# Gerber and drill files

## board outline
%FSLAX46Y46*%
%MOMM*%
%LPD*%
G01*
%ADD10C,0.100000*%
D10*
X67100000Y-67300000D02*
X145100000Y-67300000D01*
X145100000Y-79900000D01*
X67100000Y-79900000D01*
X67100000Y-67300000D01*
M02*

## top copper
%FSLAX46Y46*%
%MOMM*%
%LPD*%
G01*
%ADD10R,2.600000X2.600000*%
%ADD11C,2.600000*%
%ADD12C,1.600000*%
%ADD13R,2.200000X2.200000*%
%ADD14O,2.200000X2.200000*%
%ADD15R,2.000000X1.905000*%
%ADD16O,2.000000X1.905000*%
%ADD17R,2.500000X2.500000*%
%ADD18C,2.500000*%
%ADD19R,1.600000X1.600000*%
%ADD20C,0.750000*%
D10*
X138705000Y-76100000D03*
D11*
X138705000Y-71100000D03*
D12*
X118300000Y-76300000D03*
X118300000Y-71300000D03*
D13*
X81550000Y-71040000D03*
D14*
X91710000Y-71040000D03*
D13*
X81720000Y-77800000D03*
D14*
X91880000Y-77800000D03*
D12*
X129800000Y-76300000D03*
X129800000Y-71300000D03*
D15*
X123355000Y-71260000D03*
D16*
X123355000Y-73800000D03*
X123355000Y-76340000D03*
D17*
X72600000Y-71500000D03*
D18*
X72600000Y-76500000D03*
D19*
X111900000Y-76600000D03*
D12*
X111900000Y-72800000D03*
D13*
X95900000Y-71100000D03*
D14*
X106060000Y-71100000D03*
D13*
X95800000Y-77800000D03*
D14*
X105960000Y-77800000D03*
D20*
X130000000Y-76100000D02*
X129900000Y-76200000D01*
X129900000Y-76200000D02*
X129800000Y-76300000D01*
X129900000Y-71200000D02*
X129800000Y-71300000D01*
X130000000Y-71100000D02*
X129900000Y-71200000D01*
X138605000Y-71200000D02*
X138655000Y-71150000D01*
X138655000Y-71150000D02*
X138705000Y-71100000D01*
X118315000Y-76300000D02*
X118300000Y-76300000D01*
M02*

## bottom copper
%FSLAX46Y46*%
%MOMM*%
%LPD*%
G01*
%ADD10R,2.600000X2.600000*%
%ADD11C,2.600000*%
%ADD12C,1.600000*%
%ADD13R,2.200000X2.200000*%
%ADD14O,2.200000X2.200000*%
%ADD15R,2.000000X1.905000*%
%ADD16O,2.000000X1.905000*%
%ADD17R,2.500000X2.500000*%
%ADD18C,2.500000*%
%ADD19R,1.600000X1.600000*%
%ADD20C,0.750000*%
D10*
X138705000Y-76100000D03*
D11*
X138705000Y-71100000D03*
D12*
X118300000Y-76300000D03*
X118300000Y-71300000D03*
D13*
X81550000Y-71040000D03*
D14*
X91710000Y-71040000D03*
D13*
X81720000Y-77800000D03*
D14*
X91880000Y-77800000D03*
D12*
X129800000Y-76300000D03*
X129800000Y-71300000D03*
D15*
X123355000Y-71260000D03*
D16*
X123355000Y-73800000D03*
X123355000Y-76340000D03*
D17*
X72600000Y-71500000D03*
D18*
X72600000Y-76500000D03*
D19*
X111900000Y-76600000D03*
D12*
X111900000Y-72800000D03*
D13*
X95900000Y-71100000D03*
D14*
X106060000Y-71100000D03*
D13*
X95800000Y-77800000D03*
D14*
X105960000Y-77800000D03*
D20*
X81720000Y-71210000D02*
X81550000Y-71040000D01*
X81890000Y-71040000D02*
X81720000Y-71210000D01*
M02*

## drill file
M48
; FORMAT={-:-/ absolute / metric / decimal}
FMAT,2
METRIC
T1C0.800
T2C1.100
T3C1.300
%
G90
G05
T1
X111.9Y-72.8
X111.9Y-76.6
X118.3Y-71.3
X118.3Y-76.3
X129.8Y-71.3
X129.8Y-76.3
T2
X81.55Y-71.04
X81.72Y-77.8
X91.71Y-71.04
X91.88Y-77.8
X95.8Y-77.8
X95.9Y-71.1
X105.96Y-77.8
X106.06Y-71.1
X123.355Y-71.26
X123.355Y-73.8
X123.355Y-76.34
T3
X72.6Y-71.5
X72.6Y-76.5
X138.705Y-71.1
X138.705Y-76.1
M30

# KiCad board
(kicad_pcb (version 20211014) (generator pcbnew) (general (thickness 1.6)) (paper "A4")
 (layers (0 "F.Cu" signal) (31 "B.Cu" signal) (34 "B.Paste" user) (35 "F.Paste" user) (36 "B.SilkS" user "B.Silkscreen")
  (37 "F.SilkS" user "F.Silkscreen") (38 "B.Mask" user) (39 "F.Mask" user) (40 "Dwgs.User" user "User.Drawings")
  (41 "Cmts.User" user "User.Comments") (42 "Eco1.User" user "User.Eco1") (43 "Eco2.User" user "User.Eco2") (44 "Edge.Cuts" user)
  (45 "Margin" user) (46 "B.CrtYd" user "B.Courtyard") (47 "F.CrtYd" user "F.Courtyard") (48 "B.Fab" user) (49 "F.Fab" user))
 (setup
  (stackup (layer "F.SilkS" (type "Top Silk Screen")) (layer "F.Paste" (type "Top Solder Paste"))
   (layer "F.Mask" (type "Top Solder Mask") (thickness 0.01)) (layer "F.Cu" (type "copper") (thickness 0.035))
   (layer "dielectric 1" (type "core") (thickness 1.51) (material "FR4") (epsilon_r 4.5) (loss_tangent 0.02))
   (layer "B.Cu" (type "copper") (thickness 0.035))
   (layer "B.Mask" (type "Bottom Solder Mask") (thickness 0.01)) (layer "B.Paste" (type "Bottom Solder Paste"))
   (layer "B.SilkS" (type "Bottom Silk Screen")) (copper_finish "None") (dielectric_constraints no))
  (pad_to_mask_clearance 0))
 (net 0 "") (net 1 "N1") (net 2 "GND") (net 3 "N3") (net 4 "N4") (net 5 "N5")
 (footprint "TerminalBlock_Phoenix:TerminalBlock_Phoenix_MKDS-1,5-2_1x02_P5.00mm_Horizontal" (layer "F.Cu") (at 138.705 76.1 90)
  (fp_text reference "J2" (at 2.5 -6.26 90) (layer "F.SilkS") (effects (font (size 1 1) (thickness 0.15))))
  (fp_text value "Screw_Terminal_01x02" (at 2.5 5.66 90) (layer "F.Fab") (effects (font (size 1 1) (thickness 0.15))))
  (pad "1" thru_hole rect (at 0 0 90) (size 2.6 2.6) (drill 1.3) (layers *.Cu *.Mask) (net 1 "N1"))
  (pad "2" thru_hole circle (at 5 0 90) (size 2.6 2.6) (drill 1.3) (layers *.Cu *.Mask) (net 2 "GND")))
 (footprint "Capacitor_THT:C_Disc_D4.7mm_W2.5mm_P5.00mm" (layer "F.Cu") (at 118.3 76.3 90)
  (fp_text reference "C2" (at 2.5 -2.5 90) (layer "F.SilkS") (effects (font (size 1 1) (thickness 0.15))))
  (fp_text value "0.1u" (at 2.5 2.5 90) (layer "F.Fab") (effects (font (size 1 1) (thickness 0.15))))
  (pad "1" thru_hole circle (at 0 0 90) (size 1.6 1.6) (drill 0.8) (layers *.Cu *.Mask) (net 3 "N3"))
  (pad "2" thru_hole circle (at 5 0 90) (size 1.6 1.6) (drill 0.8) (layers *.Cu *.Mask) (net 2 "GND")))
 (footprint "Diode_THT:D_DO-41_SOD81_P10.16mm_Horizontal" (layer "F.Cu") (at 81.55 71.04)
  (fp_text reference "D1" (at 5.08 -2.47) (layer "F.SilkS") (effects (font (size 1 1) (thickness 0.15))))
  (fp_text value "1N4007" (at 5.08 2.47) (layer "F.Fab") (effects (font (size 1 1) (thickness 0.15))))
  (pad "1" thru_hole rect (at 0 0) (size 2.2 2.2) (drill 1.1) (layers *.Cu *.Mask) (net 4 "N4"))
  (pad "2" thru_hole oval (at 10.16 0) (size 2.2 2.2) (drill 1.1) (layers *.Cu *.Mask) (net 2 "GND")))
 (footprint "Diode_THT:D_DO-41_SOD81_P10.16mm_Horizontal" (layer "F.Cu") (at 81.72 77.8)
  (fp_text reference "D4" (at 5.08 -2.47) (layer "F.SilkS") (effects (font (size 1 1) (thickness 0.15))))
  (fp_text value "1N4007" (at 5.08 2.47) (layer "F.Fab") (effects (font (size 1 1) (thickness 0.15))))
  (pad "1" thru_hole rect (at 0 0) (size 2.2 2.2) (drill 1.1) (layers *.Cu *.Mask) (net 3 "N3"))
  (pad "2" thru_hole oval (at 10.16 0) (size 2.2 2.2) (drill 1.1) (layers *.Cu *.Mask) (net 4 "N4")))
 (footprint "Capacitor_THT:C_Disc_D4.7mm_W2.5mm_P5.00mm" (layer "F.Cu") (at 129.8 76.3 90)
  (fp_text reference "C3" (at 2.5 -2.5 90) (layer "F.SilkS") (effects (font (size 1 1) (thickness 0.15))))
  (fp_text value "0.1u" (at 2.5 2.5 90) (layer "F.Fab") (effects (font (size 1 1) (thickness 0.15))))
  (pad "1" thru_hole circle (at 0 0 90) (size 1.6 1.6) (drill 0.8) (layers *.Cu *.Mask) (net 1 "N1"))
  (pad "2" thru_hole circle (at 5 0 90) (size 1.6 1.6) (drill 0.8) (layers *.Cu *.Mask) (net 2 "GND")))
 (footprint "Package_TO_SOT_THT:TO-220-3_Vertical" (layer "F.Cu") (at 123.355 71.26 -90)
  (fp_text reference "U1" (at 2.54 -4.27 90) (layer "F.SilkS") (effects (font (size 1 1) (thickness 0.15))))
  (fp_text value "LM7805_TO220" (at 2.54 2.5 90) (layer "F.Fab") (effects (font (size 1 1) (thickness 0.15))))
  (pad "1" thru_hole rect (at 0 0 270) (size 1.905 2) (drill 1.1) (layers *.Cu *.Mask) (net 3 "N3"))
  (pad "2" thru_hole oval (at 2.54 0 270) (size 1.905 2) (drill 1.1) (layers *.Cu *.Mask) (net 2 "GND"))
  (pad "3" thru_hole oval (at 5.08 0 270) (size 1.905 2) (drill 1.1) (layers *.Cu *.Mask) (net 1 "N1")))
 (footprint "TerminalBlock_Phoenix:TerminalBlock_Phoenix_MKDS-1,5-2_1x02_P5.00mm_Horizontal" (layer "F.Cu") (at 72.6 71.5 -90)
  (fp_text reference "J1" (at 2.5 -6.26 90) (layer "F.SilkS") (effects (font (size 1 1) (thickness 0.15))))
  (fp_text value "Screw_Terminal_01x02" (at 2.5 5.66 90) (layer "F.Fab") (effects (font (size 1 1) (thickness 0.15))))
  (pad "1" thru_hole rect (at 0 0 270) (size 2.5 2.5) (drill 1.3) (layers *.Cu *.Mask) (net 4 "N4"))
  (pad "2" thru_hole circle (at 5 0 270) (size 2.5 2.5) (drill 1.3) (layers *.Cu *.Mask) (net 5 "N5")))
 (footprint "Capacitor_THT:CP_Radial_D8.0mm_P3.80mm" (layer "F.Cu") (at 111.9 76.6 90)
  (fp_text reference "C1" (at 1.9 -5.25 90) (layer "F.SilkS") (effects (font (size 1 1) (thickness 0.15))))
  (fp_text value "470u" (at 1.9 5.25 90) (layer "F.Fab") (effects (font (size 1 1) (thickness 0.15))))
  (pad "1" thru_hole rect (at 0 0 90) (size 1.6 1.6) (drill 0.8) (layers *.Cu *.Mask) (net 3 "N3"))
  (pad "2" thru_hole circle (at 3.8 0 90) (size 1.6 1.6) (drill 0.8) (layers *.Cu *.Mask) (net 2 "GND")))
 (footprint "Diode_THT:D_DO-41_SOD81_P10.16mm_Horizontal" (layer "F.Cu") (at 95.9 71.1)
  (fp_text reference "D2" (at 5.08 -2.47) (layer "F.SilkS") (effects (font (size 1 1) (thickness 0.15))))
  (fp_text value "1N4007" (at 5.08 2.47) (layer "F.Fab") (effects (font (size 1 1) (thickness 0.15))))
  (pad "1" thru_hole rect (at 0 0) (size 2.2 2.2) (drill 1.1) (layers *.Cu *.Mask) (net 5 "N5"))
  (pad "2" thru_hole oval (at 10.16 0) (size 2.2 2.2) (drill 1.1) (layers *.Cu *.Mask) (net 2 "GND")))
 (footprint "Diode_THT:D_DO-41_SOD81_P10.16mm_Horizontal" (layer "F.Cu") (at 95.8 77.8)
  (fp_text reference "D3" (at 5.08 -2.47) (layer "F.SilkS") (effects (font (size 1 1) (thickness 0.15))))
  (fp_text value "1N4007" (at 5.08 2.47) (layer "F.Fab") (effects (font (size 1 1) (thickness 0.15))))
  (pad "1" thru_hole rect (at 0 0) (size 2.2 2.2) (drill 1.1) (layers *.Cu *.Mask) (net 3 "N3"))
  (pad "2" thru_hole oval (at 10.16 0) (size 2.2 2.2) (drill 1.1) (layers *.Cu *.Mask) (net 5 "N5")))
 (gr_rect (start 67.1 67.3) (end 145.1 79.9) (layer "Edge.Cuts") (width 0.1) (fill none))
 (segment (start 81.72 71.21) (end 81.55 71.04) (width 0.75) (layer "B.Cu") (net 4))
 (segment (start 81.89 71.04) (end 81.72 71.21) (width 0.75) (layer "B.Cu") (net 4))
 (segment (start 130 76.1) (end 129.9 76.2) (width 0.75) (layer "F.Cu") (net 1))
 (segment (start 129.9 76.2) (end 129.8 76.3) (width 0.75) (layer "F.Cu") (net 1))
 (segment (start 129.9 71.2) (end 129.8 71.3) (width 0.75) (layer "F.Cu") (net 2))
 (segment (start 130 71.1) (end 129.9 71.2) (width 0.75) (layer "F.Cu") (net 2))
 (segment (start 138.605 71.2) (end 138.655 71.15) (width 0.75) (layer "F.Cu") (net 2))
 (segment (start 138.655 71.15) (end 138.705 71.1) (width 0.75) (layer "F.Cu") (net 2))
 (segment (start 118.315 76.3) (end 118.3 76.3) (width 0.75) (layer "F.Cu") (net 3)))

